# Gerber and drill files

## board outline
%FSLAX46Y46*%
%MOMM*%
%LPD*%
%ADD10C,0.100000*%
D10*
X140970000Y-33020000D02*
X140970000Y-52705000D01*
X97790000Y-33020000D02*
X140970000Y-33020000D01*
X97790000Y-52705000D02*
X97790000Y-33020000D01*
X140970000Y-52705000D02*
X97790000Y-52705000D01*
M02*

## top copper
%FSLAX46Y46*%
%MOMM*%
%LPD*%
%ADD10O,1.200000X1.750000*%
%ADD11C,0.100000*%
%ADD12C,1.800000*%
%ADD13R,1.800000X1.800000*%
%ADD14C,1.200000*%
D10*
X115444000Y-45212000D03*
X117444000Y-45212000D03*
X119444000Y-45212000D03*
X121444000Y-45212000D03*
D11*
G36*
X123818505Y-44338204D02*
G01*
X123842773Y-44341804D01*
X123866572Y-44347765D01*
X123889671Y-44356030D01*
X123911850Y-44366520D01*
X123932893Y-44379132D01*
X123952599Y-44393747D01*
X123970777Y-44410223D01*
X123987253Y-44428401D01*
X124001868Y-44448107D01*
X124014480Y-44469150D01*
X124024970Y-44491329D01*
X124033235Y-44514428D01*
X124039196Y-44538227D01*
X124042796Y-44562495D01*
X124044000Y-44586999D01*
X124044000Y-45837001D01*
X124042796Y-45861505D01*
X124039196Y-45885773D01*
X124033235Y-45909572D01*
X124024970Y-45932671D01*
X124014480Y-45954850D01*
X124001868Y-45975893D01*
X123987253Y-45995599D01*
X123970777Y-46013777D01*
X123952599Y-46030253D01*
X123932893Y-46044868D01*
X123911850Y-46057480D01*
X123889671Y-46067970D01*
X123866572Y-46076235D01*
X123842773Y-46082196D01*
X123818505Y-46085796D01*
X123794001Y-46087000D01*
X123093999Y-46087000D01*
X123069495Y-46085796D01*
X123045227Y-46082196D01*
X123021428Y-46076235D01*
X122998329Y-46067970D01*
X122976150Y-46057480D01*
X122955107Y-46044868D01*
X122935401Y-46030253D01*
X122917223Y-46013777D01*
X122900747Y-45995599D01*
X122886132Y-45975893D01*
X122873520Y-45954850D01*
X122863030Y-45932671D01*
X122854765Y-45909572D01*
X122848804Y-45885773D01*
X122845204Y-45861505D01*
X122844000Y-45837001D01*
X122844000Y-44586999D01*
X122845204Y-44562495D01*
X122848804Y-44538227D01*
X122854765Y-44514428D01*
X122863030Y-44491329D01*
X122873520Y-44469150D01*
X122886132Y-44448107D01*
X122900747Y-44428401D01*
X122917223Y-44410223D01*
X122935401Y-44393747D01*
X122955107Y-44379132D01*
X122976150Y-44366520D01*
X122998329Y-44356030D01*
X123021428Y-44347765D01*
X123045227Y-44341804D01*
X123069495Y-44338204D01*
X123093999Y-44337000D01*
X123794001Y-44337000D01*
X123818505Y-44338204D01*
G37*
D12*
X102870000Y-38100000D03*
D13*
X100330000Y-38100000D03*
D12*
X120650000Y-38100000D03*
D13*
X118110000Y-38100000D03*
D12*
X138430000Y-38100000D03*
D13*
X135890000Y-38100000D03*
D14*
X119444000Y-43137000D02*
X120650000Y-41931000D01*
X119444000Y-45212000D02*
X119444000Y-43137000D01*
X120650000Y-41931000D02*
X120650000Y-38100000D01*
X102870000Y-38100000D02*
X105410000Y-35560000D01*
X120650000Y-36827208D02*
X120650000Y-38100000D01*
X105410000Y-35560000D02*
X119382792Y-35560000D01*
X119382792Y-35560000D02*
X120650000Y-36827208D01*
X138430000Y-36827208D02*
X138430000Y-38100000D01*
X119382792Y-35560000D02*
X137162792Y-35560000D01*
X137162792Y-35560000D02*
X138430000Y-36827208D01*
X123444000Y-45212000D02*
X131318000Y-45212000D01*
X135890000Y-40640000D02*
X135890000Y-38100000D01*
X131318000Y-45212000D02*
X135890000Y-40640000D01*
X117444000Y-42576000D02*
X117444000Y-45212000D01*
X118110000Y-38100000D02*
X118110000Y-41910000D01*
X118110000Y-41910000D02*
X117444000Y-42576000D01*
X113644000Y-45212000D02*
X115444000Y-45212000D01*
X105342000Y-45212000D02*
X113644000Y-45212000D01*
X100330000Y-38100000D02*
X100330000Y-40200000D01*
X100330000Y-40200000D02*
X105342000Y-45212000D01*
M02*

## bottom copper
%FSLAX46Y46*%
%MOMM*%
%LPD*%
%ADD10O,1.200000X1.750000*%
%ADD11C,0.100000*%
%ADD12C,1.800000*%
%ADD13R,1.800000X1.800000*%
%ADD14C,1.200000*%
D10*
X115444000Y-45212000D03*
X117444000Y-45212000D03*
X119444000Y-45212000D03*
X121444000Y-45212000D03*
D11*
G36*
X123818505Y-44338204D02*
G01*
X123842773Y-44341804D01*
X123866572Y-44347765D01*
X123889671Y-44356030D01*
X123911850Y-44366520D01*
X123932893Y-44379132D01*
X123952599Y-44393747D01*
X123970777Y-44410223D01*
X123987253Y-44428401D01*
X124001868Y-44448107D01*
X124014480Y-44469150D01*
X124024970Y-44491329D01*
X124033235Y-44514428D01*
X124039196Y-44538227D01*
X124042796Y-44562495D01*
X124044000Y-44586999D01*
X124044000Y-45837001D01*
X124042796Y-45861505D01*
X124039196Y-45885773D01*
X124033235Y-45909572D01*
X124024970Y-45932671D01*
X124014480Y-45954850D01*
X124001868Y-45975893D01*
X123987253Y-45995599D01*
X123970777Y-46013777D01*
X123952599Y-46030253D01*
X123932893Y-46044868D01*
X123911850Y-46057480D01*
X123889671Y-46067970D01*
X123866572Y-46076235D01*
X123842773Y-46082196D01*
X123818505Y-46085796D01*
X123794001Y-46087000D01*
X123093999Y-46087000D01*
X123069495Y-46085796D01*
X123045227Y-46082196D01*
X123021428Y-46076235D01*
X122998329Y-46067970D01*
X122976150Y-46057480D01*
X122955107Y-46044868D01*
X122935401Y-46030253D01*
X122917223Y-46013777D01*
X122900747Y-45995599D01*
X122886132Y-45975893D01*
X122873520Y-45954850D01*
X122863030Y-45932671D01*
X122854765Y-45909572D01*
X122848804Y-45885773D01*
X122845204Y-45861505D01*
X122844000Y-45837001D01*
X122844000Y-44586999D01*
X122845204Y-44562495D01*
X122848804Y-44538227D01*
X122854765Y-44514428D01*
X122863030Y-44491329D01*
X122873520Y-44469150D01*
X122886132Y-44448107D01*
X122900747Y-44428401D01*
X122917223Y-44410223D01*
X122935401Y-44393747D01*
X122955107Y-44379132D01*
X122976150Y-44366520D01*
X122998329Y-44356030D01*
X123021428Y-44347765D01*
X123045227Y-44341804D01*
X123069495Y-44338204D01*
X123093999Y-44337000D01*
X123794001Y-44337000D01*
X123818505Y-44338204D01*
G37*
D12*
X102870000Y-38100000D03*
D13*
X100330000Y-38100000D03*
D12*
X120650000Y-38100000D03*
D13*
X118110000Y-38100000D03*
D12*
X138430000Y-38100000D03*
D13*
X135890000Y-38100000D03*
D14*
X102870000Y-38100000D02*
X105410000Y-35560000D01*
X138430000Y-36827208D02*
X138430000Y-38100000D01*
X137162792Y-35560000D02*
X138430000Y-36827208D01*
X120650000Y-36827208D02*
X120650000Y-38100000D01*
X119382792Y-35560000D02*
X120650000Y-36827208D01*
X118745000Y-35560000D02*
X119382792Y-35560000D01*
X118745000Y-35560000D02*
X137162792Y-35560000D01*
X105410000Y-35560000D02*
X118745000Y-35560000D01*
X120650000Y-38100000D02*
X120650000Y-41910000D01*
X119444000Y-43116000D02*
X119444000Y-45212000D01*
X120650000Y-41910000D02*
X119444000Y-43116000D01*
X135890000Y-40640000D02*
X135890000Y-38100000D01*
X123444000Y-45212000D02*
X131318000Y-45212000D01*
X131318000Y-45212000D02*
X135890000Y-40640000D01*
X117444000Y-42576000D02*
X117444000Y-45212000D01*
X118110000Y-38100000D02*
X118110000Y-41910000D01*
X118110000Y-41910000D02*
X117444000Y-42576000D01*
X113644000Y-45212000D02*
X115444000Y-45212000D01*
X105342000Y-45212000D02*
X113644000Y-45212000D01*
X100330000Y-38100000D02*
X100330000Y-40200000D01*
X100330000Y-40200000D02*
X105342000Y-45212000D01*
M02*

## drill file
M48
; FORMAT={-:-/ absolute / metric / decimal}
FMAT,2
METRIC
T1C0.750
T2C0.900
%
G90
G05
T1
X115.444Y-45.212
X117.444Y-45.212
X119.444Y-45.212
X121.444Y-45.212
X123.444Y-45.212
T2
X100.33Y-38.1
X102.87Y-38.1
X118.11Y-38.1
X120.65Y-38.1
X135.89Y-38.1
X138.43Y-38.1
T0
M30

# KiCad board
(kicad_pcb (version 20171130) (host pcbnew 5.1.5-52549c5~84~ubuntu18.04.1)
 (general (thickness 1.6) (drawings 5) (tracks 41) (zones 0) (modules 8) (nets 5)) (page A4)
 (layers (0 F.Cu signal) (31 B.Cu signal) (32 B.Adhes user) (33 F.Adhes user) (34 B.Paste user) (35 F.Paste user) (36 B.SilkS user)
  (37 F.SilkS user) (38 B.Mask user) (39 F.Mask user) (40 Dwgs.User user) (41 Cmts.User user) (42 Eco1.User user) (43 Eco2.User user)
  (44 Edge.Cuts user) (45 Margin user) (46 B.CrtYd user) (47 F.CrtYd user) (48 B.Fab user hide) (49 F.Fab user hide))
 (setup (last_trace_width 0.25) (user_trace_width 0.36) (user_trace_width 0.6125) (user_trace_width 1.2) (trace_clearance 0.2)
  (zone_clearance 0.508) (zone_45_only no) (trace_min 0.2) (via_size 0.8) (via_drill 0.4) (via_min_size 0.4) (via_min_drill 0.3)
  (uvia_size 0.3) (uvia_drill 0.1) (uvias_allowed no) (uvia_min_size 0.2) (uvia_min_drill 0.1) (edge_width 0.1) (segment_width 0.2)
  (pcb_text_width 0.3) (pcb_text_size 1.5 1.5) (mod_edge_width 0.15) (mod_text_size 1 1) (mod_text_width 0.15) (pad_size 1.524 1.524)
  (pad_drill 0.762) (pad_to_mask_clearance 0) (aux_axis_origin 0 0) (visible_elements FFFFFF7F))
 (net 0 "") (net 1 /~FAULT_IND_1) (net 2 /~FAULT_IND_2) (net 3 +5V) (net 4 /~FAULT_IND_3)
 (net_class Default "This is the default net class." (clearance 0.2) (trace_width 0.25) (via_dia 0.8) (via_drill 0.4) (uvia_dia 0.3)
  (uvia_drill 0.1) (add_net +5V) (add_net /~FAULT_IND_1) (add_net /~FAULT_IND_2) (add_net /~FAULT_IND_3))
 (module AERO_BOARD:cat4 (layer B.Cu) (at 135.255 43.815 180)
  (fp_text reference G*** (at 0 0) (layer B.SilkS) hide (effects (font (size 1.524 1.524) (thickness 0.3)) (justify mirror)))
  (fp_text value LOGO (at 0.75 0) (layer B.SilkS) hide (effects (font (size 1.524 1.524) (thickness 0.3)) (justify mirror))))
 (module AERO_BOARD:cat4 (layer B.Cu) (at 104.14 43.815 180)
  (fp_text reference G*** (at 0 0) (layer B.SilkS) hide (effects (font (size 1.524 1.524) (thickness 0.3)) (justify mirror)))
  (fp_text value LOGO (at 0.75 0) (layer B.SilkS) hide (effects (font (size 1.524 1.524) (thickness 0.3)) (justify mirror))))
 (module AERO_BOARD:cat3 (layer F.Cu) (at 119.38 39.37)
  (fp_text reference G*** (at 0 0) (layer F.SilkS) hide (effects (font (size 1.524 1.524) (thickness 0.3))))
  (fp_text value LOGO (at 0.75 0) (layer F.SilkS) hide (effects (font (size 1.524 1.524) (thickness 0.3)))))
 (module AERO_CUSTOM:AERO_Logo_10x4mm (layer B.Cu) (at 110.49 38.1 180)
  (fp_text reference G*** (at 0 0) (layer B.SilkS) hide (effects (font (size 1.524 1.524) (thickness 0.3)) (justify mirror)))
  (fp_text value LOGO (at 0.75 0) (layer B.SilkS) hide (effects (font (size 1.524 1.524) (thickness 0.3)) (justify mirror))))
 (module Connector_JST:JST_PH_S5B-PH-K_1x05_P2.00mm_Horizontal (layer B.Cu) (at 123.444 45.212 180)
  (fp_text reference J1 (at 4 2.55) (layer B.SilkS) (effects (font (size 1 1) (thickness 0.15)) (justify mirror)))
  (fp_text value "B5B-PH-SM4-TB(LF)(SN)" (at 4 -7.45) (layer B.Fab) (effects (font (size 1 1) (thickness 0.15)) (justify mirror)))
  (pad 5 thru_hole oval (at 8 0 180) (size 1.2 1.75) (drill 0.75) (layers *.Cu *.Mask) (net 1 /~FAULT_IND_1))
  (pad 4 thru_hole oval (at 6 0 180) (size 1.2 1.75) (drill 0.75) (layers *.Cu *.Mask) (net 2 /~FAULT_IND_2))
  (pad 3 thru_hole oval (at 4 0 180) (size 1.2 1.75) (drill 0.75) (layers *.Cu *.Mask) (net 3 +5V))
  (pad 2 thru_hole oval (at 2 0 180) (size 1.2 1.75) (drill 0.75) (layers *.Cu *.Mask))
  (pad 1 thru_hole roundrect (at 0 0 180) (size 1.2 1.75) (drill 0.75) (layers *.Cu *.Mask) (roundrect_rratio 0.208333)
   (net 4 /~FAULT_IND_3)))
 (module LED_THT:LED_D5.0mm (layer F.Cu) (at 100.33 38.1)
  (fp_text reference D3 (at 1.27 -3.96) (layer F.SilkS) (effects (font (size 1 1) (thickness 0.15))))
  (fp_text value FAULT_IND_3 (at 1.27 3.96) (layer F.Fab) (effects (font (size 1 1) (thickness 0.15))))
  (pad 2 thru_hole circle (at 2.54 0) (size 1.8 1.8) (drill 0.9) (layers *.Cu *.Mask) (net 3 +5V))
  (pad 1 thru_hole rect (at 0 0) (size 1.8 1.8) (drill 0.9) (layers *.Cu *.Mask) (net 1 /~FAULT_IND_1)))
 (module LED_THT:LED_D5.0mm (layer F.Cu) (at 118.11 38.1)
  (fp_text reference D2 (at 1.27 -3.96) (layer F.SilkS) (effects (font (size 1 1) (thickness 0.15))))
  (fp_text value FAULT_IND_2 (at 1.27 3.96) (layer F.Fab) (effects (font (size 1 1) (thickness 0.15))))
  (pad 2 thru_hole circle (at 2.54 0) (size 1.8 1.8) (drill 0.9) (layers *.Cu *.Mask) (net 3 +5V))
  (pad 1 thru_hole rect (at 0 0) (size 1.8 1.8) (drill 0.9) (layers *.Cu *.Mask) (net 2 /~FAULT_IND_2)))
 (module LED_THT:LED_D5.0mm (layer F.Cu) (at 135.89 38.1)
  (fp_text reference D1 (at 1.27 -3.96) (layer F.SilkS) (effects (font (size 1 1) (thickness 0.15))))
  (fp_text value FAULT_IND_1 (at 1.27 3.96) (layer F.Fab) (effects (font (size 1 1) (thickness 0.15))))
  (pad 2 thru_hole circle (at 2.54 0) (size 1.8 1.8) (drill 0.9) (layers *.Cu *.Mask) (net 3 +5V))
  (pad 1 thru_hole rect (at 0 0) (size 1.8 1.8) (drill 0.9) (layers *.Cu *.Mask) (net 4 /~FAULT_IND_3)))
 (gr_line (start 140.97 33.02) (end 140.97 52.705) (layer Edge.Cuts) (width 0.1))
 (gr_line (start 97.79 33.02) (end 140.97 33.02) (layer Edge.Cuts) (width 0.1))
 (gr_line (start 97.79 52.705) (end 97.79 33.02) (layer Edge.Cuts) (width 0.1))
 (gr_line (start 140.97 52.705) (end 97.79 52.705) (layer Edge.Cuts) (width 0.1))
 (segment (start 119.444 43.137) (end 120.65 41.931) (width 1.2) (layer F.Cu) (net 3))
 (segment (start 119.444 45.212) (end 119.444 43.137) (width 1.2) (layer F.Cu) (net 3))
 (segment (start 120.65 41.931) (end 120.65 38.1) (width 1.2) (layer F.Cu) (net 3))
 (segment (start 102.87 38.1) (end 105.41 35.56) (width 1.2) (layer F.Cu) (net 3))
 (segment (start 120.65 36.827208) (end 120.65 38.1) (width 1.2) (layer F.Cu) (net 3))
 (segment (start 105.41 35.56) (end 119.382792 35.56) (width 1.2) (layer F.Cu) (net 3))
 (segment (start 119.382792 35.56) (end 120.65 36.827208) (width 1.2) (layer F.Cu) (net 3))
 (segment (start 138.43 36.827208) (end 138.43 38.1) (width 1.2) (layer F.Cu) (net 3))
 (segment (start 119.382792 35.56) (end 137.162792 35.56) (width 1.2) (layer F.Cu) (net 3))
 (segment (start 137.162792 35.56) (end 138.43 36.827208) (width 1.2) (layer F.Cu) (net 3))
 (segment (start 102.87 38.1) (end 105.41 35.56) (width 1.2) (layer B.Cu) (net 3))
 (segment (start 138.43 36.827208) (end 138.43 38.1) (width 1.2) (layer B.Cu) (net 3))
 (segment (start 137.162792 35.56) (end 138.43 36.827208) (width 1.2) (layer B.Cu) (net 3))
 (segment (start 120.65 36.827208) (end 120.65 38.1) (width 1.2) (layer B.Cu) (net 3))
 (segment (start 119.382792 35.56) (end 120.65 36.827208) (width 1.2) (layer B.Cu) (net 3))
 (segment (start 118.745 35.56) (end 119.382792 35.56) (width 1.2) (layer B.Cu) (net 3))
 (segment (start 118.745 35.56) (end 137.162792 35.56) (width 1.2) (layer B.Cu) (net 3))
 (segment (start 105.41 35.56) (end 118.745 35.56) (width 1.2) (layer B.Cu) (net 3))
 (segment (start 120.65 38.1) (end 120.65 41.91) (width 1.2) (layer B.Cu) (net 3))
 (segment (start 119.444 43.116) (end 119.444 45.212) (width 1.2) (layer B.Cu) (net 3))
 (segment (start 120.65 41.91) (end 119.444 43.116) (width 1.2) (layer B.Cu) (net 3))
 (segment (start 135.89 40.64) (end 135.89 38.1) (width 1.2) (layer B.Cu) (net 4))
 (segment (start 123.444 45.212) (end 131.318 45.212) (width 1.2) (layer B.Cu) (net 4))
 (segment (start 131.318 45.212) (end 135.89 40.64) (width 1.2) (layer B.Cu) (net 4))
 (segment (start 123.444 45.212) (end 131.318 45.212) (width 1.2) (layer F.Cu) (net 4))
 (segment (start 135.89 40.64) (end 135.89 38.1) (width 1.2) (layer F.Cu) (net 4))
 (segment (start 131.318 45.212) (end 135.89 40.64) (width 1.2) (layer F.Cu) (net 4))
 (segment (start 117.444 42.576) (end 117.444 45.212) (width 1.2) (layer F.Cu) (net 2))
 (segment (start 118.11 38.1) (end 118.11 41.91) (width 1.2) (layer F.Cu) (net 2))
 (segment (start 118.11 41.91) (end 117.444 42.576) (width 1.2) (layer F.Cu) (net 2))
 (segment (start 117.444 42.576) (end 117.444 45.212) (width 1.2) (layer B.Cu) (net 2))
 (segment (start 118.11 38.1) (end 118.11 41.91) (width 1.2) (layer B.Cu) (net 2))
 (segment (start 118.11 41.91) (end 117.444 42.576) (width 1.2) (layer B.Cu) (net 2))
 (segment (start 113.644 45.212) (end 115.444 45.212) (width 1.2) (layer F.Cu) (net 1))
 (segment (start 105.342 45.212) (end 113.644 45.212) (width 1.2) (layer F.Cu) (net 1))
 (segment (start 100.33 38.1) (end 100.33 40.2) (width 1.2) (layer F.Cu) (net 1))
 (segment (start 100.33 40.2) (end 105.342 45.212) (width 1.2) (layer F.Cu) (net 1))
 (segment (start 113.644 45.212) (end 115.444 45.212) (width 1.2) (layer B.Cu) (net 1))
 (segment (start 105.342 45.212) (end 113.644 45.212) (width 1.2) (layer B.Cu) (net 1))
 (segment (start 100.33 38.1) (end 100.33 40.2) (width 1.2) (layer B.Cu) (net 1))
 (segment (start 100.33 40.2) (end 105.342 45.212) (width 1.2) (layer B.Cu) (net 1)))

